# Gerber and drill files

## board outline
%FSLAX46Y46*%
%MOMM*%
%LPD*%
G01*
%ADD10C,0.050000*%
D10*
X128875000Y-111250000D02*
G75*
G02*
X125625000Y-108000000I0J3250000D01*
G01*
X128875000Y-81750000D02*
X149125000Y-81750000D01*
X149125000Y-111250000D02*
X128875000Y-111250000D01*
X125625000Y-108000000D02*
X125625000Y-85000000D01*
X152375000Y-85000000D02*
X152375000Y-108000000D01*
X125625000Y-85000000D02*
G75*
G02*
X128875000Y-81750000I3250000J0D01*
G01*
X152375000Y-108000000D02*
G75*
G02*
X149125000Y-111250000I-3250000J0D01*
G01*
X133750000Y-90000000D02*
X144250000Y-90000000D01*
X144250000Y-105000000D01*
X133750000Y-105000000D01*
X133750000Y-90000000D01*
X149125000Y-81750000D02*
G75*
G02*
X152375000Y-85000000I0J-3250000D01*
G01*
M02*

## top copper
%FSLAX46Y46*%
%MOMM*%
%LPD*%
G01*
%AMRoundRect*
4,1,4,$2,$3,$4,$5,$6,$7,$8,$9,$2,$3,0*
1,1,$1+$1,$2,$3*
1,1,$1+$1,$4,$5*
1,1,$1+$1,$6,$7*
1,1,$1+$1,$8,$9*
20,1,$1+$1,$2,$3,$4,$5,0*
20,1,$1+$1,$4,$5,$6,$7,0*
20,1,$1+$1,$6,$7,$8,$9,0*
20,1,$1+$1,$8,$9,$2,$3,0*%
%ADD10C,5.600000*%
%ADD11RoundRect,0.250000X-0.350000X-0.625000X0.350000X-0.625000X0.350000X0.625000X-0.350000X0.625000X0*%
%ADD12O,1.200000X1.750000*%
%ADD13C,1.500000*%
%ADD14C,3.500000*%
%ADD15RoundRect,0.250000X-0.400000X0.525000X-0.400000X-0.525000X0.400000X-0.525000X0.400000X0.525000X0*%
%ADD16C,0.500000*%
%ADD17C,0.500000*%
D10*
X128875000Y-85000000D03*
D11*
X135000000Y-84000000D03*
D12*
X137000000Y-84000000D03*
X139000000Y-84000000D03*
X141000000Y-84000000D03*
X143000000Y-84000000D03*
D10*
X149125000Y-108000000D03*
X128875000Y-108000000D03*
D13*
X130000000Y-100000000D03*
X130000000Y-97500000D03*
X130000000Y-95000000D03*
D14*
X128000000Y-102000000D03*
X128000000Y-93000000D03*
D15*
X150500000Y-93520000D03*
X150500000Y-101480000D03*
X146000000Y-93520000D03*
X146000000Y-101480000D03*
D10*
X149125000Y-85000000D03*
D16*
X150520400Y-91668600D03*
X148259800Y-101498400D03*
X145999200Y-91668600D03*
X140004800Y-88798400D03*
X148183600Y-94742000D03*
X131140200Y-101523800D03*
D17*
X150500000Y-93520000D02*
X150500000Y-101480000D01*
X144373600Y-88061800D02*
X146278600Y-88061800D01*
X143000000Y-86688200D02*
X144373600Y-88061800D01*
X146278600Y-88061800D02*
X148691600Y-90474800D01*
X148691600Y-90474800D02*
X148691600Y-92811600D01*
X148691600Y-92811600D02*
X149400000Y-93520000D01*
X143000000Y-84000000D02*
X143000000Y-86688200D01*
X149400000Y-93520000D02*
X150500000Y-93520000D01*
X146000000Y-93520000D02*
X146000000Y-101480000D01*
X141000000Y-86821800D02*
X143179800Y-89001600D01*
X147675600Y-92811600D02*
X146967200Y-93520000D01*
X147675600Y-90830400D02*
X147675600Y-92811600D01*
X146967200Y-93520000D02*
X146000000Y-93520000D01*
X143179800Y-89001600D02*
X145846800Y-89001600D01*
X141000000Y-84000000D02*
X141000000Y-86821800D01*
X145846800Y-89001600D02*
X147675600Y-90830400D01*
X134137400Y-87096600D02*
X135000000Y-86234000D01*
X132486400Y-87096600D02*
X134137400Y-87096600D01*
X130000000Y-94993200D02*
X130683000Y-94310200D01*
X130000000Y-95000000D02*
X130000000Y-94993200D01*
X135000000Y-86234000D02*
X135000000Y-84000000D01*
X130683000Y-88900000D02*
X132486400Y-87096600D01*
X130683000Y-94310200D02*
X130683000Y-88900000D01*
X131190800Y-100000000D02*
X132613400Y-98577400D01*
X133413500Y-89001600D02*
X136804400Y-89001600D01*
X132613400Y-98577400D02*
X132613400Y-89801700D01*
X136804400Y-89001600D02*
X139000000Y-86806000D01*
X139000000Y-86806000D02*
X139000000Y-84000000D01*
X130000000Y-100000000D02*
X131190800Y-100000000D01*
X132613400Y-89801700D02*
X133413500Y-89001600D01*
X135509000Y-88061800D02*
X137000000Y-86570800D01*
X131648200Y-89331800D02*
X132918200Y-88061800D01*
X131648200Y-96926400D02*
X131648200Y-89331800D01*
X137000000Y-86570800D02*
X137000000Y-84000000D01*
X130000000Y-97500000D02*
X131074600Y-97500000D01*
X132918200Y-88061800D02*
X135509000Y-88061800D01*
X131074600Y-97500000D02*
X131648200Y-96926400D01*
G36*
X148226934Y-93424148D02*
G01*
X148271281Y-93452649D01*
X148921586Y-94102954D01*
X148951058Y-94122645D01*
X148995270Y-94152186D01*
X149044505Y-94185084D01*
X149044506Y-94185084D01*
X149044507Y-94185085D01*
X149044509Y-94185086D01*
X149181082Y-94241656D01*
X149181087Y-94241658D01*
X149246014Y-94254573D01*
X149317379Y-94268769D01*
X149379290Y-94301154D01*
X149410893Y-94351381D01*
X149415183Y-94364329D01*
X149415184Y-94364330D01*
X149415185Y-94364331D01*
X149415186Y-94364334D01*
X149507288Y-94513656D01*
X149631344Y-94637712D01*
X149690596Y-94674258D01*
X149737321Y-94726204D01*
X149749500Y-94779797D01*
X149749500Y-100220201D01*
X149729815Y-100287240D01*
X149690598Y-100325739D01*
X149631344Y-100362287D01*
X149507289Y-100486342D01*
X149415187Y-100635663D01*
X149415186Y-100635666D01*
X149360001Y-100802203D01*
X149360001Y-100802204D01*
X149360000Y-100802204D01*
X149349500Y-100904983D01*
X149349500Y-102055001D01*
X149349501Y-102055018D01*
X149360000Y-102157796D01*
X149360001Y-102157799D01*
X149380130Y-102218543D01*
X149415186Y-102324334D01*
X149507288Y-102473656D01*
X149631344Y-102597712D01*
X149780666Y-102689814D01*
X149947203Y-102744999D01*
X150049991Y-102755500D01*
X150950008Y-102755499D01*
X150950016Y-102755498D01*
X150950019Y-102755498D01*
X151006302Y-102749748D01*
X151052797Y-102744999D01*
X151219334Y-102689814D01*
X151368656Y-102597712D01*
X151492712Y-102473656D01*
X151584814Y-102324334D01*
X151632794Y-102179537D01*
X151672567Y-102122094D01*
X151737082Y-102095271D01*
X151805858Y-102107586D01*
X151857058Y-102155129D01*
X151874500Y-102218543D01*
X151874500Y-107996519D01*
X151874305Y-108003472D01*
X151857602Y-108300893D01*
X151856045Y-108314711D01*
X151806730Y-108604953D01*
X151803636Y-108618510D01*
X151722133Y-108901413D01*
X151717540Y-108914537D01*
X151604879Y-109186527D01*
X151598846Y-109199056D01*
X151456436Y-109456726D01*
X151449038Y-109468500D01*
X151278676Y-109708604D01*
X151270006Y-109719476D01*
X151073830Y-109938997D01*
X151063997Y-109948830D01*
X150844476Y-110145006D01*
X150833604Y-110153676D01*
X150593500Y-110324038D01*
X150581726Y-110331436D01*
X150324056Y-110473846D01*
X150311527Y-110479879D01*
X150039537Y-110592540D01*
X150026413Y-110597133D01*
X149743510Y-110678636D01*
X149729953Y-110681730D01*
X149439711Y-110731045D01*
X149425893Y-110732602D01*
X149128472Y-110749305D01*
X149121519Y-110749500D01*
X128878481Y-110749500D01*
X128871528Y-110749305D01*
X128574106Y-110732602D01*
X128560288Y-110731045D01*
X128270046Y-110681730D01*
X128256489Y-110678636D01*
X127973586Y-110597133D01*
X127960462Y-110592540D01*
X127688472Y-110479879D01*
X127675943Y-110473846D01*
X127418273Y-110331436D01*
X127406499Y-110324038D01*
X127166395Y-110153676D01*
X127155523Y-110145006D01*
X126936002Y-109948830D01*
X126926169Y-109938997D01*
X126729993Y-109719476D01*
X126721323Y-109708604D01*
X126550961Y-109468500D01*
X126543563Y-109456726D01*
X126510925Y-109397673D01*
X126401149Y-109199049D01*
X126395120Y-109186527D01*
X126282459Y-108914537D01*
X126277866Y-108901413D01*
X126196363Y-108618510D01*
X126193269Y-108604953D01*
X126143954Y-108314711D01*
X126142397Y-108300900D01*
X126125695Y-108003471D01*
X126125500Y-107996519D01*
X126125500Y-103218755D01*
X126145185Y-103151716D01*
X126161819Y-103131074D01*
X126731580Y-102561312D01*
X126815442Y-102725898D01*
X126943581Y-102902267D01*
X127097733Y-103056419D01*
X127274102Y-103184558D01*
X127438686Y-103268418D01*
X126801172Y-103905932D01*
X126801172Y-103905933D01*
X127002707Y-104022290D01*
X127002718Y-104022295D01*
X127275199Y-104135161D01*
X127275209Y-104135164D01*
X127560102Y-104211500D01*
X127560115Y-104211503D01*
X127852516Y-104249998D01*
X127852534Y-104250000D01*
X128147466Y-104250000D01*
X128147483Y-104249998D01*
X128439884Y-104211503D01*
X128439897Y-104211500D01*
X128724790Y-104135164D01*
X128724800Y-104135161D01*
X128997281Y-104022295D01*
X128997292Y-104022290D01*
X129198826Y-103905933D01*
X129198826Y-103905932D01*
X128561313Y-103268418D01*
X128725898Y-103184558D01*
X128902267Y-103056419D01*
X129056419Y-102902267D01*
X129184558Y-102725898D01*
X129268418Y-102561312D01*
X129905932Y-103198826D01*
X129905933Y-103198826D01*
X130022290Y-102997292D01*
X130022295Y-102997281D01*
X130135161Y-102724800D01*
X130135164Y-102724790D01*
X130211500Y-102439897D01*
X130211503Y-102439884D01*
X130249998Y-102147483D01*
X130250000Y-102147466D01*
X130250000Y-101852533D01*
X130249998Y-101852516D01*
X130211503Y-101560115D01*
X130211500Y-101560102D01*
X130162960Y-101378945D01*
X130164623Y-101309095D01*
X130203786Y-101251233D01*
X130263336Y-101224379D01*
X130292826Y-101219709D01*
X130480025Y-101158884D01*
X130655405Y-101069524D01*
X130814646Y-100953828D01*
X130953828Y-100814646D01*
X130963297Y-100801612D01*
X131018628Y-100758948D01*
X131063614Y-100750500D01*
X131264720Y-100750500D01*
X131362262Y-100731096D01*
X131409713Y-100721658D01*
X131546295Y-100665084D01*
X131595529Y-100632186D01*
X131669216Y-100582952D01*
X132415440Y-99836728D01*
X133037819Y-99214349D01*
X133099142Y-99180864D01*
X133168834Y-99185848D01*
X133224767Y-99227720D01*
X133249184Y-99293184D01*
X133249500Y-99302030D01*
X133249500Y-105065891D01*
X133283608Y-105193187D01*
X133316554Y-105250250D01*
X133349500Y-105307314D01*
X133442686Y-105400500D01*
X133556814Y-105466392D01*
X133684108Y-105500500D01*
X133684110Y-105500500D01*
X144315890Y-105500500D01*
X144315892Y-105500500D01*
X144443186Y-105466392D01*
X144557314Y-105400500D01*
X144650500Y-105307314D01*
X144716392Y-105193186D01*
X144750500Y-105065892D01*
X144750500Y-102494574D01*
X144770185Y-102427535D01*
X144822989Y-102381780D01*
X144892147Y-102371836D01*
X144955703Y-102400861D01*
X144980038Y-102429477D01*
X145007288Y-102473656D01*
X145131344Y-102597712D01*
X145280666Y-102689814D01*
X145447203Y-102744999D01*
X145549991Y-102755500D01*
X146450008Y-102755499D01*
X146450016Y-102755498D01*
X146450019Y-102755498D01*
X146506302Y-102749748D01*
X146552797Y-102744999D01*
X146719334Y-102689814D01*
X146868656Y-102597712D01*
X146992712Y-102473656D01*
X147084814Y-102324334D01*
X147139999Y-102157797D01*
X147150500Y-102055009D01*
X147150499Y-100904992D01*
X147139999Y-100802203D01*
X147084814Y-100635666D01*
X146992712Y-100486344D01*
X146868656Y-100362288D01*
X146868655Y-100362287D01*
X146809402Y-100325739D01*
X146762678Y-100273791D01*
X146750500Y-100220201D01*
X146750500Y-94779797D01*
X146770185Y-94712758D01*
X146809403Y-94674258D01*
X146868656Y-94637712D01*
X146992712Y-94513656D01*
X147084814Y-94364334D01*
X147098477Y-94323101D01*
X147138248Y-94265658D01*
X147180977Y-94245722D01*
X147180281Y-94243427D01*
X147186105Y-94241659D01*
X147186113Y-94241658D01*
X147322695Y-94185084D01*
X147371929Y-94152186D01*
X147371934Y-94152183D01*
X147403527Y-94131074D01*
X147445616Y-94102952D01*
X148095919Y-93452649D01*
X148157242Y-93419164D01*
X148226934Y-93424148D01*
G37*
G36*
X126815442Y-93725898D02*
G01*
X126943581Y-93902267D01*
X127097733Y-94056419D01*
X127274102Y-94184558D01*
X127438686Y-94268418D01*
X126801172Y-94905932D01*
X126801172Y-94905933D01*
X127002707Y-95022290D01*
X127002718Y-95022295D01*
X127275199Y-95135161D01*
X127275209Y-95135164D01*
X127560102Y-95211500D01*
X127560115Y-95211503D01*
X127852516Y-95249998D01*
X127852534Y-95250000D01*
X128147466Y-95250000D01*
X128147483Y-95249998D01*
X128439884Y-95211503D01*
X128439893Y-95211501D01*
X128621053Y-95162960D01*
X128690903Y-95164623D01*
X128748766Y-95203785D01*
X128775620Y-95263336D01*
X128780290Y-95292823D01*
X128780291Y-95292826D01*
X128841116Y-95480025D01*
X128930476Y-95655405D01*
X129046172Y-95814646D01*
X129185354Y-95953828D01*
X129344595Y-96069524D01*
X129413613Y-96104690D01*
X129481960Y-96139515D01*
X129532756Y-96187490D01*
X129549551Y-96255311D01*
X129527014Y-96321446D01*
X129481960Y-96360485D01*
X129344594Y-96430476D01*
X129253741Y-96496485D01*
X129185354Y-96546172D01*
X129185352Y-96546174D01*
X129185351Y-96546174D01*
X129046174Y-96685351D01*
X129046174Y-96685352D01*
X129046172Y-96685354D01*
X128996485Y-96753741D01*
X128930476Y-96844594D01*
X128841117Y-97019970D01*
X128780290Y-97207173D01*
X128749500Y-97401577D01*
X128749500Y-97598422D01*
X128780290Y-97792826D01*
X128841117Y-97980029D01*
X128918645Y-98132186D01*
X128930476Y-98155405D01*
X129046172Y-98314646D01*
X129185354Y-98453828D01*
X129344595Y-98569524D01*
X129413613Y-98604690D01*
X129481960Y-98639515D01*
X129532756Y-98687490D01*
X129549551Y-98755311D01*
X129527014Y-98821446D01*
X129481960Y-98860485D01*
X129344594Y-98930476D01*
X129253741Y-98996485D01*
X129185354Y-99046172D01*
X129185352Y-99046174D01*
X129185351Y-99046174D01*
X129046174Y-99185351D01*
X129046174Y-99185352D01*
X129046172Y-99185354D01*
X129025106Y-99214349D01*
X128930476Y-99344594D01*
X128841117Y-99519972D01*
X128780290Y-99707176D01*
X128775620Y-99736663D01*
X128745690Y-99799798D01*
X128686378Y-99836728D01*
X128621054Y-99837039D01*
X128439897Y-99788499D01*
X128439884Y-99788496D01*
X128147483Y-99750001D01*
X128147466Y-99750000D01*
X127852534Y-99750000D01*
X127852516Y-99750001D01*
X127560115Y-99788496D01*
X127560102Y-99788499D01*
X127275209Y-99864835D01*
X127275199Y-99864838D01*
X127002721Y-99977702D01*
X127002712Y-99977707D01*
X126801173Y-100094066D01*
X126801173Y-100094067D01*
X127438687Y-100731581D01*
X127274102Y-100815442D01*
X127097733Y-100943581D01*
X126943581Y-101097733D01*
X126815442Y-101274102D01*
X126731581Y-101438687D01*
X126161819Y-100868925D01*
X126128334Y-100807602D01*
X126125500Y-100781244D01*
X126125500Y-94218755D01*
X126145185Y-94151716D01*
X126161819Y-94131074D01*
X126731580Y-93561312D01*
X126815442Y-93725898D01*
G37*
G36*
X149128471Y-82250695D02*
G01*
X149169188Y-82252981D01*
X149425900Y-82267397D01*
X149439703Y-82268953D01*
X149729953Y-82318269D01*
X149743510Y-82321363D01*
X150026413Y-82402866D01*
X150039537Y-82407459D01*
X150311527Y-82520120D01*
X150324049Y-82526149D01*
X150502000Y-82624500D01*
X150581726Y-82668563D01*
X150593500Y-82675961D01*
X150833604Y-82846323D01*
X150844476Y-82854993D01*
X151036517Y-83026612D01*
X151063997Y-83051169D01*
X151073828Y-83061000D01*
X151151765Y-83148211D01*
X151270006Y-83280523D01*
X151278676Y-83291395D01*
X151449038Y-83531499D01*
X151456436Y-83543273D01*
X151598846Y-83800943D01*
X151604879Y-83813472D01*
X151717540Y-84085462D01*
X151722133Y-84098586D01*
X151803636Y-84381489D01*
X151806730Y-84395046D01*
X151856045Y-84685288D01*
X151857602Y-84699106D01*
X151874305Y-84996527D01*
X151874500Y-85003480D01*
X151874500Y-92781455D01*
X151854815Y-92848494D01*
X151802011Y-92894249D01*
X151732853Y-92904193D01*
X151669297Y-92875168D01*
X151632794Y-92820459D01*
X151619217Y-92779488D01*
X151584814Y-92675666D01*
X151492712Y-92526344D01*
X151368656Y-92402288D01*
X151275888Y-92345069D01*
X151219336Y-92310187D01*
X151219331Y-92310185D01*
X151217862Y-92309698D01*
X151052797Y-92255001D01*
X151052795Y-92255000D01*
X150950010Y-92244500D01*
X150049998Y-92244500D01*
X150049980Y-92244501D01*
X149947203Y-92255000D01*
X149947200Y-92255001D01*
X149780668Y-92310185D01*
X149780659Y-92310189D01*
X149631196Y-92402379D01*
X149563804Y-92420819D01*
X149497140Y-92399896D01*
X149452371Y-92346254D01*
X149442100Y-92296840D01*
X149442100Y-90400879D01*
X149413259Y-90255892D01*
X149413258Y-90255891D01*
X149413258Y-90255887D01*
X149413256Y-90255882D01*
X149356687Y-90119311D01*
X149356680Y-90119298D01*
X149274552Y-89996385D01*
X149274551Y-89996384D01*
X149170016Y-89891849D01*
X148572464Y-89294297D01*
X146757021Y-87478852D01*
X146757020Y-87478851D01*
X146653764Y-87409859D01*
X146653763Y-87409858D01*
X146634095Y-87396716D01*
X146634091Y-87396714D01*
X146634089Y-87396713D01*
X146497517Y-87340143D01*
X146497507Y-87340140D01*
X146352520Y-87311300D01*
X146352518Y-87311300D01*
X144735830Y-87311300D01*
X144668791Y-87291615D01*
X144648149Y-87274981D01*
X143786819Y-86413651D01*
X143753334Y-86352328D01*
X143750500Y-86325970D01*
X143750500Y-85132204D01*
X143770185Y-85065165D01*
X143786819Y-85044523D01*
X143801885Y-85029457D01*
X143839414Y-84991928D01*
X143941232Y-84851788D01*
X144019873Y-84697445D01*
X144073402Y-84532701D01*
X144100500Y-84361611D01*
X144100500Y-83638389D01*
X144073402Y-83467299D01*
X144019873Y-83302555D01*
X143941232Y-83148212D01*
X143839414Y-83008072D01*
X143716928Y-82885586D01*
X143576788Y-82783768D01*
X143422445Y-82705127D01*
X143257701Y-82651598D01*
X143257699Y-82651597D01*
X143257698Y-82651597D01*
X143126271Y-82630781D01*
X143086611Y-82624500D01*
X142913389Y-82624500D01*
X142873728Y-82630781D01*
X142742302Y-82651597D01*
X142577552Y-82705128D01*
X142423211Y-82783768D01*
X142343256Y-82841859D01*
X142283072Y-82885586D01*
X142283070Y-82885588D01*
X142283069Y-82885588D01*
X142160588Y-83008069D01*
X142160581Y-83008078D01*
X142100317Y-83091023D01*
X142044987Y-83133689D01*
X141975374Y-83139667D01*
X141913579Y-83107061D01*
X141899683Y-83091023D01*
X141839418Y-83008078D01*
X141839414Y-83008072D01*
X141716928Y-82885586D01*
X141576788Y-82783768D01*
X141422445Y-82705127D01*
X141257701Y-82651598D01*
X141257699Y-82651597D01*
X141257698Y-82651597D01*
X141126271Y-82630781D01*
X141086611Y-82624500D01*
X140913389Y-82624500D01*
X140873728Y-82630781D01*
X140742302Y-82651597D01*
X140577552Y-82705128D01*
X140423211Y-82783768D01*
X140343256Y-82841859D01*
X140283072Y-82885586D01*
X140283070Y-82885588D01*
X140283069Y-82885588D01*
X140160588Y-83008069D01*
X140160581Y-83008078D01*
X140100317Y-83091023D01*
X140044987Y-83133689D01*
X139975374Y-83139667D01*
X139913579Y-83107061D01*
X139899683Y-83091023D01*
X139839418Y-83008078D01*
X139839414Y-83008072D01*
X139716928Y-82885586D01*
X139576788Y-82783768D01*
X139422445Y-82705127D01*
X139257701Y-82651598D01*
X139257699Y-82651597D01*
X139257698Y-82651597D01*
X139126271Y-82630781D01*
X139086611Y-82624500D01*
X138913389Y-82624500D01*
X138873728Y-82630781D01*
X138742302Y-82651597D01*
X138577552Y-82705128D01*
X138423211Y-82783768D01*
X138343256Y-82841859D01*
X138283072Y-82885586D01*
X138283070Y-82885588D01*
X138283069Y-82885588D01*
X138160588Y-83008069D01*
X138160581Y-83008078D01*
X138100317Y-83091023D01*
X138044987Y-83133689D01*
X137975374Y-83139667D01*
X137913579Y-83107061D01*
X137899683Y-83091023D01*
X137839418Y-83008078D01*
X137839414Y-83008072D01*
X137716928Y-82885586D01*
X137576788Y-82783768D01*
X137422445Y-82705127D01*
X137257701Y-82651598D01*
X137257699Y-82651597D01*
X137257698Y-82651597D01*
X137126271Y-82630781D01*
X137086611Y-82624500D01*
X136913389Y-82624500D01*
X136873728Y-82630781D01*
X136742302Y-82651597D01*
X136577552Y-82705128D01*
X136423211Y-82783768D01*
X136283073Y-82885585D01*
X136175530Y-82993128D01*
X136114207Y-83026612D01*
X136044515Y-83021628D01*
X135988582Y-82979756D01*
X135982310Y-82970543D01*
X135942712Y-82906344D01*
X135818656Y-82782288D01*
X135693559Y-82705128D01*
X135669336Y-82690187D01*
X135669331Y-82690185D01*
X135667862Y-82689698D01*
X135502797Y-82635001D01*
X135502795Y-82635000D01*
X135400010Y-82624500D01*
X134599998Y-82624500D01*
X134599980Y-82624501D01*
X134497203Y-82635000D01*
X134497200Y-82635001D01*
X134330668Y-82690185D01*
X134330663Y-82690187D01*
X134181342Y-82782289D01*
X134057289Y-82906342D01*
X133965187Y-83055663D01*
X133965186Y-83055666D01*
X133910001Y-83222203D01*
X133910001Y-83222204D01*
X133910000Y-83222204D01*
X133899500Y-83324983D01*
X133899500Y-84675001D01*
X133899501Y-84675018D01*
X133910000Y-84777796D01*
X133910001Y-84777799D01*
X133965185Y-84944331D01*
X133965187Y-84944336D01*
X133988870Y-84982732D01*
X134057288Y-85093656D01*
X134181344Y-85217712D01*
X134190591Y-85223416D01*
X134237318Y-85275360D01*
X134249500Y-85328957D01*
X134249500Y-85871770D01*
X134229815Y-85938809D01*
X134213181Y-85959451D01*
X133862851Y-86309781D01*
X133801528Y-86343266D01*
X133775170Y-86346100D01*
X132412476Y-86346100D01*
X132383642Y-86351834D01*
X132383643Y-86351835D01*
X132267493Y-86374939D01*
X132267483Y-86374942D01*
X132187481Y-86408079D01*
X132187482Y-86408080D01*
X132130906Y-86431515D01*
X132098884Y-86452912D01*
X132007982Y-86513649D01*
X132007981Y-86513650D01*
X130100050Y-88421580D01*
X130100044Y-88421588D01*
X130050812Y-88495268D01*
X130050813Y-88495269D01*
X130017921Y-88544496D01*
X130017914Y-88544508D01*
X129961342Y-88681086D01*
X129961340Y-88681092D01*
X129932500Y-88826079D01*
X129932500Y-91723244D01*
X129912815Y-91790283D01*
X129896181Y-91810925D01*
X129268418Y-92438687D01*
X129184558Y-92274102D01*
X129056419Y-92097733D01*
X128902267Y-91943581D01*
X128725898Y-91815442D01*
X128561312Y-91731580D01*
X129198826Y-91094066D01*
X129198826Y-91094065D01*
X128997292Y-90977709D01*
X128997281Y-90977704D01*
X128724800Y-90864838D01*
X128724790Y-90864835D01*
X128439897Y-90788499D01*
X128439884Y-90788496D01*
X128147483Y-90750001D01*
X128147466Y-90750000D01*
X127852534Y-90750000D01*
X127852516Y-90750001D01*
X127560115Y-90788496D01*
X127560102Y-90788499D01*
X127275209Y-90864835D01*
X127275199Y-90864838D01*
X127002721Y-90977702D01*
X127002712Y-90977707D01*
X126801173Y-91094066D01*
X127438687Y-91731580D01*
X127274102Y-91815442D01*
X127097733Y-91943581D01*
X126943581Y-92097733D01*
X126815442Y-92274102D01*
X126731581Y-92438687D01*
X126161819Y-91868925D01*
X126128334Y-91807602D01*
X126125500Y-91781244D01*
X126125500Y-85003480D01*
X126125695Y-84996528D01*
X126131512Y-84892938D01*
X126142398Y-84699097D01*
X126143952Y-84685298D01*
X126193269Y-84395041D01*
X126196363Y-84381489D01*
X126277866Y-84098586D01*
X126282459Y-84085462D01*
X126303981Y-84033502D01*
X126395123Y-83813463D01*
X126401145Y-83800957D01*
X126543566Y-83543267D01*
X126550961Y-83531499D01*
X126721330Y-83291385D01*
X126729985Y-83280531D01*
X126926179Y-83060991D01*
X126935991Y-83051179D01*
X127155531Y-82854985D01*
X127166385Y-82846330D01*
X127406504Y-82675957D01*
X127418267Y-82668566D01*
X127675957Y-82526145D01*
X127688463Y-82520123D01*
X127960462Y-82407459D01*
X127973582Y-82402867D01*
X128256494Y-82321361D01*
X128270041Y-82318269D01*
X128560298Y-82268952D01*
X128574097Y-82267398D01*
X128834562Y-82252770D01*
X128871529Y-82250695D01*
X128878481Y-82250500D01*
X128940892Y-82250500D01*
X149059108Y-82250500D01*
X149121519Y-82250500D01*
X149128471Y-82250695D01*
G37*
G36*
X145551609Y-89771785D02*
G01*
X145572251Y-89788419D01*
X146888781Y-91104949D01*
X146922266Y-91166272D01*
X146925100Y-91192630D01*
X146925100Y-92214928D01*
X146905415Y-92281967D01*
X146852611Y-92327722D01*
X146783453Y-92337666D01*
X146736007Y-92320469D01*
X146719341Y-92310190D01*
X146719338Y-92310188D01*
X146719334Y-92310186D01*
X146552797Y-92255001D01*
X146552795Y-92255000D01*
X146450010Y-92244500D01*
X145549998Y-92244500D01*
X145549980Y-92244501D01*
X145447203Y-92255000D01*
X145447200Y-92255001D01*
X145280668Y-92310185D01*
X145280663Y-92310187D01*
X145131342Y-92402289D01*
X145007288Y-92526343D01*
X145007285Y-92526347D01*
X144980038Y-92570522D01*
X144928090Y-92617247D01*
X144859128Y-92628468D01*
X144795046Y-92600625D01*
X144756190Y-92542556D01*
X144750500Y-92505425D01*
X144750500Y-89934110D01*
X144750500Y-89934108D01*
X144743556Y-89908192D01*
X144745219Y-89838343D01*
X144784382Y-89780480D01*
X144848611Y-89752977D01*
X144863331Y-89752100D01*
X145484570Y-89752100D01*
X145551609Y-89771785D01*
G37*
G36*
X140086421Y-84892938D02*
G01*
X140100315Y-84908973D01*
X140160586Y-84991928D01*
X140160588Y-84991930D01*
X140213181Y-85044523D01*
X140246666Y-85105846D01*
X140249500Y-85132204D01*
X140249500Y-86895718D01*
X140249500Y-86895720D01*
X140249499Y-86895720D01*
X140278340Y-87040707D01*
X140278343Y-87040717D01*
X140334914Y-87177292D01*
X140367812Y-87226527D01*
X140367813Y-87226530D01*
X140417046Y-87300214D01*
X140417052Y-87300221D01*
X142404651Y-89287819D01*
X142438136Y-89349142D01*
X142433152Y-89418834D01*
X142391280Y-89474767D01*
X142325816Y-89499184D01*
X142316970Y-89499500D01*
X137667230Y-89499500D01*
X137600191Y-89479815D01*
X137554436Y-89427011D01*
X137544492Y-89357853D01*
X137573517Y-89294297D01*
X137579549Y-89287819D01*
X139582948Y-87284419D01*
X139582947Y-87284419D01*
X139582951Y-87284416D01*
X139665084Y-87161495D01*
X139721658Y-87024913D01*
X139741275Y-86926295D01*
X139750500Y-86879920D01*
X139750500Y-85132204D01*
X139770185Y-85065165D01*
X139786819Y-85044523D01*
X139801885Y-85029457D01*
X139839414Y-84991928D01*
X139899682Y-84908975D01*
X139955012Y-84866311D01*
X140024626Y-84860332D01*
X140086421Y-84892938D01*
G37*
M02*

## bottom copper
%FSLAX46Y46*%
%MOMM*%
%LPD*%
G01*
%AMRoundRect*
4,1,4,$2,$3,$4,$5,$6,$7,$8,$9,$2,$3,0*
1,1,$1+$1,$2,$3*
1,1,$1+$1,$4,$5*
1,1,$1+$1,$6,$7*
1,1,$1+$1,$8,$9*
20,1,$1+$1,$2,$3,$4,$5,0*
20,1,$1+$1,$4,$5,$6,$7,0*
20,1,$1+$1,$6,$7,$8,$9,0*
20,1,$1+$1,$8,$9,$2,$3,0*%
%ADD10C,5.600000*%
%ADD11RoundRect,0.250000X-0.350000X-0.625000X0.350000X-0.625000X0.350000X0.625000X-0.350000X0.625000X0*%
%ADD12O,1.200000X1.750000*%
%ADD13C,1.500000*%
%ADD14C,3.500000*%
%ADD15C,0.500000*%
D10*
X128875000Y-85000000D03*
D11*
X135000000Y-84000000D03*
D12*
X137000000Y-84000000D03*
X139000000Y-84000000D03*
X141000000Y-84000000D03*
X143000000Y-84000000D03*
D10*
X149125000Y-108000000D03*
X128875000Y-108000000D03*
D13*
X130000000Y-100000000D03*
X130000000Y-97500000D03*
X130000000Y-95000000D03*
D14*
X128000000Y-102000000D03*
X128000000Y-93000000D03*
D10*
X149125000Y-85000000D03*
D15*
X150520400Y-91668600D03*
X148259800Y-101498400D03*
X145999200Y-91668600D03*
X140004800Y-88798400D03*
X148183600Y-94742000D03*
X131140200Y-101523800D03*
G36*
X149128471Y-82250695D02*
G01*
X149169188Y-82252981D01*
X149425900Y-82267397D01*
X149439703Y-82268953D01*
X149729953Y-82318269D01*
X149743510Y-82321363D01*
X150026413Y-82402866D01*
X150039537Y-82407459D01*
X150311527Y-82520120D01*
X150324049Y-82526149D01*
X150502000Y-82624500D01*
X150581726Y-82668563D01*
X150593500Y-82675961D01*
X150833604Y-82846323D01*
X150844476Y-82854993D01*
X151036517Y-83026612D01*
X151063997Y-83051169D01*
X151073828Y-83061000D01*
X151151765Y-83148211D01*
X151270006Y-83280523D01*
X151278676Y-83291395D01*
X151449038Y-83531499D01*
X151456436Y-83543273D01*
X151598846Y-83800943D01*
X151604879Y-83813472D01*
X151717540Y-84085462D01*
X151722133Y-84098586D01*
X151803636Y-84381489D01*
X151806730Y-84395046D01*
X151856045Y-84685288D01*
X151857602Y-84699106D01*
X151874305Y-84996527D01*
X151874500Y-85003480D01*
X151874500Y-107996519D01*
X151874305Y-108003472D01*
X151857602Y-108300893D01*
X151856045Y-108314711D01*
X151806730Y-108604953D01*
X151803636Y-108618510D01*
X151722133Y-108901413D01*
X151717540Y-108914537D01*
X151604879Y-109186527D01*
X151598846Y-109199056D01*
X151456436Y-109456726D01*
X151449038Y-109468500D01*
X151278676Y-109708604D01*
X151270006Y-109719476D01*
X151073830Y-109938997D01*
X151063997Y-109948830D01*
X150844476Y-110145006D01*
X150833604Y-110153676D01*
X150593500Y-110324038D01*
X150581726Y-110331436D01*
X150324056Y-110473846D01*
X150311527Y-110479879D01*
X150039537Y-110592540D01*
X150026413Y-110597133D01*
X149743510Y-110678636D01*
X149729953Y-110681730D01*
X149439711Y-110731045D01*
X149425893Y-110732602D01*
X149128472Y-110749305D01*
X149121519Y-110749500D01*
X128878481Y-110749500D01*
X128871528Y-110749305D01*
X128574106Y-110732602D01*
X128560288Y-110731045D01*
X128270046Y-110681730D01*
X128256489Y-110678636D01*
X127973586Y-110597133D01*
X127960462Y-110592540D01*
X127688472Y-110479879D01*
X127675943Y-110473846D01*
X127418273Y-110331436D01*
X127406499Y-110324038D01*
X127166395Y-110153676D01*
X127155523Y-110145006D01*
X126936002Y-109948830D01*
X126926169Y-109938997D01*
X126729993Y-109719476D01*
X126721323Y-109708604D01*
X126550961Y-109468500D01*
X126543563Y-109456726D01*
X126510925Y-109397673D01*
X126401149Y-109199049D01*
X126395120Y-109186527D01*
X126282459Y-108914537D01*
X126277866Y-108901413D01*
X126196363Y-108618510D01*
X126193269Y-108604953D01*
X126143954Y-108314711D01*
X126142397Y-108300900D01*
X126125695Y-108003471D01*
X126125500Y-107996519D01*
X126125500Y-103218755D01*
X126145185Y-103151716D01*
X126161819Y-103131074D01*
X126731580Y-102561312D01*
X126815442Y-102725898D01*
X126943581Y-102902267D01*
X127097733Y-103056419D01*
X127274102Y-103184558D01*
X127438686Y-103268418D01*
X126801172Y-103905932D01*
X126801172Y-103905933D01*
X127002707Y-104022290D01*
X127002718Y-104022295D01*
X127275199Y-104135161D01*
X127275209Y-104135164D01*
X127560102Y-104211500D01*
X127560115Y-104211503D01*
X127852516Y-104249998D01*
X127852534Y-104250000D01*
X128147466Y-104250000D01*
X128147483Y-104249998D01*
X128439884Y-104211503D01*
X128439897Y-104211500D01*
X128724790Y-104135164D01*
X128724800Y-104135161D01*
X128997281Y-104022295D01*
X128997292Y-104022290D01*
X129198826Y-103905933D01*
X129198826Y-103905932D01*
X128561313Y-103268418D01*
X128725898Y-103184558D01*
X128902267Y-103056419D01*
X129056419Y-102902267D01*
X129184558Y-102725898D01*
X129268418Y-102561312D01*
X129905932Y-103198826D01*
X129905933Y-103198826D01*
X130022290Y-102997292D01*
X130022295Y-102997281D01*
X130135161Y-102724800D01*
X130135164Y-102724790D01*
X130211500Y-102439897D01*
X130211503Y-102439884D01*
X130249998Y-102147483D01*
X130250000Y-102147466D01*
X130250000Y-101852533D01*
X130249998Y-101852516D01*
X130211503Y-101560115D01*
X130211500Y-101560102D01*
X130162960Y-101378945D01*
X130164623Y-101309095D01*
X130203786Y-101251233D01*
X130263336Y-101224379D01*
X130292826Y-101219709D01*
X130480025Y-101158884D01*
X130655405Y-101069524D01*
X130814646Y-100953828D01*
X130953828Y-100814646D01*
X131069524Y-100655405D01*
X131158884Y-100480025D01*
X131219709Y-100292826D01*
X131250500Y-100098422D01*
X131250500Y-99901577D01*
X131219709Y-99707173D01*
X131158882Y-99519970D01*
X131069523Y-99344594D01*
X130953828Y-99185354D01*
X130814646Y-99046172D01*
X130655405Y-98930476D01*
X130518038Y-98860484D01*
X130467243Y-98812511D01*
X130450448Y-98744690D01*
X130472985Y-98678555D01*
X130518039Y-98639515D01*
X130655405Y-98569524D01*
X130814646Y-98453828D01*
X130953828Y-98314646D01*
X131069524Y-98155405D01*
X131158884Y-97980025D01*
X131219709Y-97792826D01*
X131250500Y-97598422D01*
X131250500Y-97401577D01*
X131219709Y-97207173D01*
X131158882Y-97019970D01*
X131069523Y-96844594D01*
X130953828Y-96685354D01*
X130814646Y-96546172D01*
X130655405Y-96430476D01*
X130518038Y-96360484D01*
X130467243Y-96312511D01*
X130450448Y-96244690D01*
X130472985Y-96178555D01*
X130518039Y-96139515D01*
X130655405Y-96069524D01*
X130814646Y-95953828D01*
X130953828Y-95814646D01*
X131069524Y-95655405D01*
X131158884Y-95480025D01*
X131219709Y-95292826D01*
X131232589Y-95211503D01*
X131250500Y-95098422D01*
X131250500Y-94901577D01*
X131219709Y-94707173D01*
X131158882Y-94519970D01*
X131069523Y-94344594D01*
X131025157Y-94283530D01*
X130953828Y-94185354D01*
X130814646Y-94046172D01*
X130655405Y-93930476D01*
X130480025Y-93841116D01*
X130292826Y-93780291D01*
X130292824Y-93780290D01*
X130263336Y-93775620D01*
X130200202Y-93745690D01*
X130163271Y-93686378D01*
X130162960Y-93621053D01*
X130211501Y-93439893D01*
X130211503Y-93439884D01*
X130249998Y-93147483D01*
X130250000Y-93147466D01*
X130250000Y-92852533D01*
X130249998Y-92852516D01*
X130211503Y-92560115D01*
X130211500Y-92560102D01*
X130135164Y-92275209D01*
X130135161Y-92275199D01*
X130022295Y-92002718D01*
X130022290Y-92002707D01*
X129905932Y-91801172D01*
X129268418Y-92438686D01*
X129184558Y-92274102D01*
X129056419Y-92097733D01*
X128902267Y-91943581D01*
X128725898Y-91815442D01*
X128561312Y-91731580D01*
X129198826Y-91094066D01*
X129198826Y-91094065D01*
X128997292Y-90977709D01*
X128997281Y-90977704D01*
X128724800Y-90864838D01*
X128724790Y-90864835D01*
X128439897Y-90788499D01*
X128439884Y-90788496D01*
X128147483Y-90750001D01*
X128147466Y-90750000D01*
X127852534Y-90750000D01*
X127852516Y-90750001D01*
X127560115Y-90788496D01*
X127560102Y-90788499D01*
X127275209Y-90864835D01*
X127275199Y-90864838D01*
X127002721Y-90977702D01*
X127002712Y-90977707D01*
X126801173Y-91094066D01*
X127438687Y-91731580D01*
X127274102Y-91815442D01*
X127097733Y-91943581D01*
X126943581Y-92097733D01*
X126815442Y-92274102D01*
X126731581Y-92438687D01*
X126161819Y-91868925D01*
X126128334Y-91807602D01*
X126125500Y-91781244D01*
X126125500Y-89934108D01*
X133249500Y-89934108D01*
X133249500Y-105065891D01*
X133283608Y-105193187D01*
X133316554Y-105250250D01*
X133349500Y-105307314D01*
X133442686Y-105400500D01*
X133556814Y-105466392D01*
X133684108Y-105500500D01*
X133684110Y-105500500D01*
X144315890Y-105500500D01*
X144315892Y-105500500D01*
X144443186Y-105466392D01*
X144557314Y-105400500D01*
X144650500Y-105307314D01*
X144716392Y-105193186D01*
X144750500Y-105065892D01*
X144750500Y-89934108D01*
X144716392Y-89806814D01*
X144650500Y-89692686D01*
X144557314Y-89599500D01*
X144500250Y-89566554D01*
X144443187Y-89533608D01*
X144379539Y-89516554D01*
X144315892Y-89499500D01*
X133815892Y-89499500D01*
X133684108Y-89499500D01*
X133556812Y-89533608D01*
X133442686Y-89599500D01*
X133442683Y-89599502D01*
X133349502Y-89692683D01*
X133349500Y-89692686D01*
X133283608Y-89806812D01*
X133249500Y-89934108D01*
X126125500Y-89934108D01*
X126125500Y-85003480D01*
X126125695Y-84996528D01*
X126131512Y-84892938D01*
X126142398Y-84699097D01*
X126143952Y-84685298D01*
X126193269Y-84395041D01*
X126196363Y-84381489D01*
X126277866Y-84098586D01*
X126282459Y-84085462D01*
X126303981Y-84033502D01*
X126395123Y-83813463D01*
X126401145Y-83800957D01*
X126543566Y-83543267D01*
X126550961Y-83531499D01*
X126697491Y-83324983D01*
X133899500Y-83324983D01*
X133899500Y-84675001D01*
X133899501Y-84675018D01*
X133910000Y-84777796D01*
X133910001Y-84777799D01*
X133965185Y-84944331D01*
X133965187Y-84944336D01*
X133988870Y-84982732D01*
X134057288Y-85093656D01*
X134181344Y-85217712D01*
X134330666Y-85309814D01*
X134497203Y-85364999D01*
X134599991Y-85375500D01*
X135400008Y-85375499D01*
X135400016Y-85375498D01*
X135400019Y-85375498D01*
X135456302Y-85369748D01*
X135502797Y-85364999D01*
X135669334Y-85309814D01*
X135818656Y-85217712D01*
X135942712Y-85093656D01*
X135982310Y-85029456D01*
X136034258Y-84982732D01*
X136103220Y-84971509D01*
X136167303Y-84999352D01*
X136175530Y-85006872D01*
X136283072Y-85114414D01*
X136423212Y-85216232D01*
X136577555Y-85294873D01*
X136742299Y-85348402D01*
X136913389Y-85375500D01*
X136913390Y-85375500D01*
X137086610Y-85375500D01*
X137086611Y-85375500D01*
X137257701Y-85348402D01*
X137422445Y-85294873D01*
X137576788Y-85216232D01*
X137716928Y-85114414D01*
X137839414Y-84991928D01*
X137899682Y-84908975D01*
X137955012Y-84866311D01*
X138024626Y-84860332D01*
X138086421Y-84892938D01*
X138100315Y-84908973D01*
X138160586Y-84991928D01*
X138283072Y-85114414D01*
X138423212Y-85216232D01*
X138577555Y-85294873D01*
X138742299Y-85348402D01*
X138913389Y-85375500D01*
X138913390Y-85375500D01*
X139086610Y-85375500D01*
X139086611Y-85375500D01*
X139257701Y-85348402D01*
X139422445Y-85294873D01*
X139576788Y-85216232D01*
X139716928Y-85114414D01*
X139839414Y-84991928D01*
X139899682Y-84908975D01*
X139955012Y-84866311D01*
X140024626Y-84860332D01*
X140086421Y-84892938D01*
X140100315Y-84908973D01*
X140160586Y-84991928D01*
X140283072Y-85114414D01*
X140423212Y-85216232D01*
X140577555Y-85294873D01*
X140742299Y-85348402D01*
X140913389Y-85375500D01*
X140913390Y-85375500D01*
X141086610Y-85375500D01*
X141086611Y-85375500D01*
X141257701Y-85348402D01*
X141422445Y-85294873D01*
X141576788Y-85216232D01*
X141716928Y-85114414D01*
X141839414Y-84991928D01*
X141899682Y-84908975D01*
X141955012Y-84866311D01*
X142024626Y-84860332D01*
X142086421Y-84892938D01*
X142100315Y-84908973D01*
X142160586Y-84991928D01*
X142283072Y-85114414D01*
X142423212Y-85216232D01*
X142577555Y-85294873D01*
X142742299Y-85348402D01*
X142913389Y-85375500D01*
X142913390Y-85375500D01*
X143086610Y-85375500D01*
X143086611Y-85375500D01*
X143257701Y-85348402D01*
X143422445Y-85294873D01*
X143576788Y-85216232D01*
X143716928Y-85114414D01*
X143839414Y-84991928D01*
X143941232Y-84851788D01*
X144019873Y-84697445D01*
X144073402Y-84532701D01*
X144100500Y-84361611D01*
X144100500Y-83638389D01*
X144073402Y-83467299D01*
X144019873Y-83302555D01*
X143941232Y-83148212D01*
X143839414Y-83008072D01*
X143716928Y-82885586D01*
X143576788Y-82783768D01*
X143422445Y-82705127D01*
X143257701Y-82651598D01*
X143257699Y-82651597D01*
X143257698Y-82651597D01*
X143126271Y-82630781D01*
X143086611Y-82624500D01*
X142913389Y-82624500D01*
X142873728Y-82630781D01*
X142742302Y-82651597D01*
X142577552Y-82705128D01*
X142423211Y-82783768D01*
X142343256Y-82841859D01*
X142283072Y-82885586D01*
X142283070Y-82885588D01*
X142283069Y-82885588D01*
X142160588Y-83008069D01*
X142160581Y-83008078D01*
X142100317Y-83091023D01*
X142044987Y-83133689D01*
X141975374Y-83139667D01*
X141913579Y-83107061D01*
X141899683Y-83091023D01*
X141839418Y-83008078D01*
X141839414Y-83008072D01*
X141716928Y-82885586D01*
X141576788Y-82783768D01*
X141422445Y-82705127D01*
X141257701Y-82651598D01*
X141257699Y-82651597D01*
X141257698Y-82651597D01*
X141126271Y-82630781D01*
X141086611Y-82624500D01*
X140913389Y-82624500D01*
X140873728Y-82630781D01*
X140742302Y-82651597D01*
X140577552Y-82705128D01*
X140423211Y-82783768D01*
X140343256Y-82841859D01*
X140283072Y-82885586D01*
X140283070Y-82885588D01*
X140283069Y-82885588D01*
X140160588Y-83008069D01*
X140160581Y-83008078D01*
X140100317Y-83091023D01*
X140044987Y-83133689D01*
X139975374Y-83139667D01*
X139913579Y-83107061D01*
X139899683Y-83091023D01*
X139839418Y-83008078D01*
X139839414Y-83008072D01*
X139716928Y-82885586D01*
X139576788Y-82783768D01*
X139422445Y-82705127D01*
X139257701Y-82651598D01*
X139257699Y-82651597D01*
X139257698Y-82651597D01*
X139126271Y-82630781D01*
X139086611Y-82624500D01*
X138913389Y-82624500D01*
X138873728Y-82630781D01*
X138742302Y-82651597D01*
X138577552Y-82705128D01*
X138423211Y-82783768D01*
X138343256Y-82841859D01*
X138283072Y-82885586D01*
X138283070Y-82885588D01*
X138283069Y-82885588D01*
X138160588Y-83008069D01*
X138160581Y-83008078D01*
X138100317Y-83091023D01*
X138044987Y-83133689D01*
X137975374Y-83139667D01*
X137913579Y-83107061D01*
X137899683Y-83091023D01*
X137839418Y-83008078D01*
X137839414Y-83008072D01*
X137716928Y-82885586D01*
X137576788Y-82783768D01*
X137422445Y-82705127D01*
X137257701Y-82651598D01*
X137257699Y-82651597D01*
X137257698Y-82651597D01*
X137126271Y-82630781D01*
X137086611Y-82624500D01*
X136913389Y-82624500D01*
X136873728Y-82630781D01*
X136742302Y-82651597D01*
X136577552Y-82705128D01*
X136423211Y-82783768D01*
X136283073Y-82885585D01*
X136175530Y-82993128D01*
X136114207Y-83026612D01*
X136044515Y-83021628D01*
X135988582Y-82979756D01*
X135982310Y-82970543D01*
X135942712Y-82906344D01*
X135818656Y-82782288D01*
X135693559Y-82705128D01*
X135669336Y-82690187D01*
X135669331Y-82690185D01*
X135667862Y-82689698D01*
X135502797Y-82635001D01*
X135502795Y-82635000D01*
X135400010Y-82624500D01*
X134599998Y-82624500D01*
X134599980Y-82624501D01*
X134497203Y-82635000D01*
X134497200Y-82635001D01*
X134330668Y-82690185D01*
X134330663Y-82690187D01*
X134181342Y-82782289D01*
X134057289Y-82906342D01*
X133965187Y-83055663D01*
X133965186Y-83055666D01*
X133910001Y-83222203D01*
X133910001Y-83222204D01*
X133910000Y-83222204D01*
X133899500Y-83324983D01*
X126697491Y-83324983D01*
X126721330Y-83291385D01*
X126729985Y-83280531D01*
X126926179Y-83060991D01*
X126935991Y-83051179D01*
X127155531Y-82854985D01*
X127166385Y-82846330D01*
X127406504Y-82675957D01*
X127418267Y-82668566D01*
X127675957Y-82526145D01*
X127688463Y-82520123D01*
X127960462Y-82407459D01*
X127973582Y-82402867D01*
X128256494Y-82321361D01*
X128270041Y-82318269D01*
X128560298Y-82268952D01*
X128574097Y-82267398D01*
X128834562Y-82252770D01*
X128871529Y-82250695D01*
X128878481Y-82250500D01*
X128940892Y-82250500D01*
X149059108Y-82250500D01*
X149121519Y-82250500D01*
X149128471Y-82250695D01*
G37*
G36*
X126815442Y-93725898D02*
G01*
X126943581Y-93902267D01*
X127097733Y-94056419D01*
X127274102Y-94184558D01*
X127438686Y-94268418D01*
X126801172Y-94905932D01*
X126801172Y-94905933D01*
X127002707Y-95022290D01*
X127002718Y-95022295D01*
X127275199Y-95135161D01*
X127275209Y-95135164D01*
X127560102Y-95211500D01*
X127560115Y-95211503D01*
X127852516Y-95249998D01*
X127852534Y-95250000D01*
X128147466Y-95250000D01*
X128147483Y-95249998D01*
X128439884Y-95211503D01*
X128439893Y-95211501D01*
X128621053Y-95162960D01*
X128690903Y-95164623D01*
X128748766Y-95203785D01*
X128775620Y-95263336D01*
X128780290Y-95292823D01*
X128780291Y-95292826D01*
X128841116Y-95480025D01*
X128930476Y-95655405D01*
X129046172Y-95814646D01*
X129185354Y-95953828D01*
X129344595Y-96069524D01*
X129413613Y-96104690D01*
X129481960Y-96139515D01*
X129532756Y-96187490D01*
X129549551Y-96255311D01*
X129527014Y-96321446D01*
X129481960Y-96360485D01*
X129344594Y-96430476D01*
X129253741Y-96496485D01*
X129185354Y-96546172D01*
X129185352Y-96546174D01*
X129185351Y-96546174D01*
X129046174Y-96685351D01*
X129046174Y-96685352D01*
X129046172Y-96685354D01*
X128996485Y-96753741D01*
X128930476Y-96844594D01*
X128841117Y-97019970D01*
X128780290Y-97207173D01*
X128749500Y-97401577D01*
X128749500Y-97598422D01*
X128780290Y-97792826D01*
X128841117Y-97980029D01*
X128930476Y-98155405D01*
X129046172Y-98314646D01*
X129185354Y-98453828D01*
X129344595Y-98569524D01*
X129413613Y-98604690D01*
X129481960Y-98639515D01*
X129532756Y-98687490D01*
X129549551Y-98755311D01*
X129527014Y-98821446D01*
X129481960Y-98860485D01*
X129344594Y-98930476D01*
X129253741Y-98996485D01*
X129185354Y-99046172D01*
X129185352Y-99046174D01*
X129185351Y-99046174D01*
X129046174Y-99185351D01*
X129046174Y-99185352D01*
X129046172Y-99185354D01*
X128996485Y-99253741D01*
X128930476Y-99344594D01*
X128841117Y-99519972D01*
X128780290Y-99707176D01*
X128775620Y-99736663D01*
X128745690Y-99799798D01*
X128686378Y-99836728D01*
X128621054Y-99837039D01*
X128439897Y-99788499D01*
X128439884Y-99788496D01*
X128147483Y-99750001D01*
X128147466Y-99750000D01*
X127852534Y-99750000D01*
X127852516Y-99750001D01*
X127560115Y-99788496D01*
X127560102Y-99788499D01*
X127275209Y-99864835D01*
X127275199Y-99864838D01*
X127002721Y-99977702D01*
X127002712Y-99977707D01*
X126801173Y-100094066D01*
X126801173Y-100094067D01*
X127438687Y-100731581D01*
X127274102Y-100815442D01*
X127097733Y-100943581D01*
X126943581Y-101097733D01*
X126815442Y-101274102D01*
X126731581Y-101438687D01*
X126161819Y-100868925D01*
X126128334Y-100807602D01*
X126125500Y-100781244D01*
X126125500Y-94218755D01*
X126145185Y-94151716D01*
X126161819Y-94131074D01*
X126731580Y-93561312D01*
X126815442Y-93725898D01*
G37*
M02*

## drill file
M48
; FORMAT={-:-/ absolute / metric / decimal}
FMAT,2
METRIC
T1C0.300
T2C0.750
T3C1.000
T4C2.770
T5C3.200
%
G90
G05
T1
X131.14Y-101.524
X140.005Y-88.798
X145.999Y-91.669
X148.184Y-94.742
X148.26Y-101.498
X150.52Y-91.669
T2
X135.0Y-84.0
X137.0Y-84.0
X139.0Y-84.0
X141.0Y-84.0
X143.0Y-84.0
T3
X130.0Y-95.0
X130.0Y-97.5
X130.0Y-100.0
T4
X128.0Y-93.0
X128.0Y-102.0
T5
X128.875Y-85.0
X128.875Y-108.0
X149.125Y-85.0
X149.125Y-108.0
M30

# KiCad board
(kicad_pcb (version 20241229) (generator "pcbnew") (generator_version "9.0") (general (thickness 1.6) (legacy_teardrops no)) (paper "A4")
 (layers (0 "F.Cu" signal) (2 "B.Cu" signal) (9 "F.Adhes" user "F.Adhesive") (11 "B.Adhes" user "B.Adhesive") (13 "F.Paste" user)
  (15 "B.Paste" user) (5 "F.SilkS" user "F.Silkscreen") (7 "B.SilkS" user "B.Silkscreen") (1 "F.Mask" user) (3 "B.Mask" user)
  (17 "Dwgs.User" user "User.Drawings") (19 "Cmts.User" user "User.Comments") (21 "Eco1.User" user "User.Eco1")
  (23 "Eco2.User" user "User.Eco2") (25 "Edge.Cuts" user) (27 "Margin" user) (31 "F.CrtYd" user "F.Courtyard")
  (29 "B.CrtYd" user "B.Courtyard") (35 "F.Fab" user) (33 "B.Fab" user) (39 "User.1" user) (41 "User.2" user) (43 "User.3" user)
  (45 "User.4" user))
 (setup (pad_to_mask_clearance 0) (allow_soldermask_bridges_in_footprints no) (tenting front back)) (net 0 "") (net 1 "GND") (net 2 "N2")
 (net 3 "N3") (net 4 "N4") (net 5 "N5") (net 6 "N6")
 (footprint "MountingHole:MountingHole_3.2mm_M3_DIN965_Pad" (layer "F.Cu") (at 128.875 85)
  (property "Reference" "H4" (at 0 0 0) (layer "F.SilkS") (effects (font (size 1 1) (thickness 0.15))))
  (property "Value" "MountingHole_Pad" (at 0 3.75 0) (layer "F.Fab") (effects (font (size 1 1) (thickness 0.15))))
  (pad "1" thru_hole circle (at 0 0) (size 5.6 5.6) (drill 3.2) (layers "*.Cu" "*.Mask") (remove_unused_layers no) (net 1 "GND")
   (zone_connect 2)))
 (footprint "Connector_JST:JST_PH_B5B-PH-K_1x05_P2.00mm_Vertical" (layer "F.Cu") (at 135 84)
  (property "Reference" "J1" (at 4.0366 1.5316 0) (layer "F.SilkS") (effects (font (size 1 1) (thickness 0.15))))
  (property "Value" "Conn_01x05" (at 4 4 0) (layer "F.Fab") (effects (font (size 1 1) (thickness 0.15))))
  (pad "1" thru_hole roundrect (at 0 0) (size 1.2 1.75) (drill 0.75) (layers "*.Cu" "*.Mask") (remove_unused_layers no)
   (roundrect_rratio 0.208333) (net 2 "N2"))
  (pad "2" thru_hole oval (at 2 0) (size 1.2 1.75) (drill 0.75) (layers "*.Cu" "*.Mask") (remove_unused_layers no) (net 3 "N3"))
  (pad "3" thru_hole oval (at 4 0) (size 1.2 1.75) (drill 0.75) (layers "*.Cu" "*.Mask") (remove_unused_layers no) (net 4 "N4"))
  (pad "4" thru_hole oval (at 6 0) (size 1.2 1.75) (drill 0.75) (layers "*.Cu" "*.Mask") (remove_unused_layers no) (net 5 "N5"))
  (pad "5" thru_hole oval (at 8 0) (size 1.2 1.75) (drill 0.75) (layers "*.Cu" "*.Mask") (remove_unused_layers no) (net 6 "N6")))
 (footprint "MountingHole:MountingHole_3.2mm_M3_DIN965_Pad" (layer "F.Cu") (at 149.125 108)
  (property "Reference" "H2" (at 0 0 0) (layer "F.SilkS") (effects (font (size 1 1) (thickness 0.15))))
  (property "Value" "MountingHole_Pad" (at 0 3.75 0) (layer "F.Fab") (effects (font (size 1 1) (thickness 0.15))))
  (pad "1" thru_hole circle (at 0 0) (size 5.6 5.6) (drill 3.2) (layers "*.Cu" "*.Mask") (remove_unused_layers no) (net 1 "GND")
   (zone_connect 2)))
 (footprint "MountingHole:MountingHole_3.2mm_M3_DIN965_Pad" (layer "F.Cu") (at 128.875 108)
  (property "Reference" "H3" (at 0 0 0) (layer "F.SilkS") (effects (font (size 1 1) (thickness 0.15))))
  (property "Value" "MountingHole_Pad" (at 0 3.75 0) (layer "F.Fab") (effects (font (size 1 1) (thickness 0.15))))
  (pad "1" thru_hole circle (at 0 0) (size 5.6 5.6) (drill 3.2) (layers "*.Cu" "*.Mask") (remove_unused_layers no) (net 1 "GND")
   (zone_connect 2)))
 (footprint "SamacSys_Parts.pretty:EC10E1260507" (layer "F.Cu") (at 130 100 90)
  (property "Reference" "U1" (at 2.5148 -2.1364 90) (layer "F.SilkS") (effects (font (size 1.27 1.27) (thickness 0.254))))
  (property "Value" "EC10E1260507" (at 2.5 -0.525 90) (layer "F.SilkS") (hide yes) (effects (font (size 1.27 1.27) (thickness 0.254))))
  (pad "A1" thru_hole circle (at 0 0 90) (size 1.5 1.5) (drill 1) (layers "*.Cu" "*.Mask") (remove_unused_layers no) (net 4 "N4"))
  (pad "B1" thru_hole circle (at 2.5 0 90) (size 1.5 1.5) (drill 1) (layers "*.Cu" "*.Mask") (remove_unused_layers no) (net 3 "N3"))
  (pad "C1" thru_hole circle (at 5 0 90) (size 1.5 1.5) (drill 1) (layers "*.Cu" "*.Mask") (remove_unused_layers no) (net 2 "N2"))
  (pad "MH1" thru_hole circle (at -2 -2 90) (size 3.5 3.5) (drill 2.77) (layers "*.Cu" "*.Mask") (remove_unused_layers no) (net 1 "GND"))
  (pad "MH2" thru_hole circle (at 7 -2 90) (size 3.5 3.5) (drill 2.77) (layers "*.Cu" "*.Mask") (remove_unused_layers no) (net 1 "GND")))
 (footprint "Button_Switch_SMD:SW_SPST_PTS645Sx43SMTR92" (layer "F.Cu") (at 148.25 97.5 -90)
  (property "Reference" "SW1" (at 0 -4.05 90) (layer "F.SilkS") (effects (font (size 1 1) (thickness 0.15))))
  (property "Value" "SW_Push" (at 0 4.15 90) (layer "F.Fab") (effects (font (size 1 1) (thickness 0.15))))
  (pad "1" smd roundrect (at -3.98 -2.25 270) (size 1.55 1.3) (layers "F.Cu" "F.Mask" "F.Paste") (roundrect_rratio 0.1923076923)
   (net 6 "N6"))
  (pad "1" smd roundrect (at 3.98 -2.25 270) (size 1.55 1.3) (layers "F.Cu" "F.Mask" "F.Paste") (roundrect_rratio 0.1923076923) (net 6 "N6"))
  (pad "2" smd roundrect (at -3.98 2.25 270) (size 1.55 1.3) (layers "F.Cu" "F.Mask" "F.Paste") (roundrect_rratio 0.1923076923) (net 5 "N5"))
  (pad "2" smd roundrect (at 3.98 2.25 270) (size 1.55 1.3) (layers "F.Cu" "F.Mask" "F.Paste") (roundrect_rratio 0.1923076923) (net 5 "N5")))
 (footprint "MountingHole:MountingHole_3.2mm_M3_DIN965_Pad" (layer "F.Cu") (at 149.125 85)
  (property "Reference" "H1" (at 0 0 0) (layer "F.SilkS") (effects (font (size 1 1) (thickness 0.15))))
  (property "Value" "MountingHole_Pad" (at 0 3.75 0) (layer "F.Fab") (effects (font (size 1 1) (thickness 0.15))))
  (pad "1" thru_hole circle (at 0 0) (size 5.6 5.6) (drill 3.2) (layers "*.Cu" "*.Mask") (remove_unused_layers no) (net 1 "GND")
   (zone_connect 2)))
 (gr_arc (start 128.875 111.25) (mid 126.576903 110.298097) (end 125.625 108) (stroke (width 0.05) (type solid)) (layer "Edge.Cuts"))
 (gr_line (start 128.875 81.75) (end 149.125 81.75) (stroke (width 0.05) (type solid)) (layer "Edge.Cuts"))
 (gr_line (start 149.125 111.25) (end 128.875 111.25) (stroke (width 0.05) (type default)) (layer "Edge.Cuts"))
 (gr_line (start 125.625 108) (end 125.625 85) (stroke (width 0.05) (type default)) (layer "Edge.Cuts"))
 (gr_line (start 152.375 85) (end 152.375 108) (stroke (width 0.05) (type solid)) (layer "Edge.Cuts"))
 (gr_arc (start 125.625 85) (mid 126.576903 82.701903) (end 128.875 81.75) (stroke (width 0.05) (type solid)) (layer "Edge.Cuts"))
 (gr_arc (start 152.375 108) (mid 151.423097 110.298097) (end 149.125 111.25) (stroke (width 0.05) (type solid)) (layer "Edge.Cuts"))
 (gr_rect (start 133.75 90) (end 144.25 105) (stroke (width 0.05) (type solid)) (fill no) (layer "Edge.Cuts"))
 (gr_arc (start 149.125 81.75) (mid 151.423097 82.701903) (end 152.375 85) (stroke (width 0.05) (type solid)) (layer "Edge.Cuts"))
 (segment (start 150.5 93.52) (end 150.5 101.48) (width 0.5) (layer "F.Cu") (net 6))
 (segment (start 144.3736 88.0618) (end 146.2786 88.0618) (width 0.5) (layer "F.Cu") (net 6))
 (segment (start 143 86.6882) (end 144.3736 88.0618) (width 0.5) (layer "F.Cu") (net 6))
 (segment (start 146.2786 88.0618) (end 148.6916 90.4748) (width 0.5) (layer "F.Cu") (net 6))
 (segment (start 148.6916 90.4748) (end 148.6916 92.8116) (width 0.5) (layer "F.Cu") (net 6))
 (segment (start 148.6916 92.8116) (end 149.4 93.52) (width 0.5) (layer "F.Cu") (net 6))
 (segment (start 143 84) (end 143 86.6882) (width 0.5) (layer "F.Cu") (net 6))
 (segment (start 149.4 93.52) (end 150.5 93.52) (width 0.5) (layer "F.Cu") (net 6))
 (segment (start 146 93.52) (end 146 101.48) (width 0.5) (layer "F.Cu") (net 5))
 (segment (start 141 86.8218) (end 143.1798 89.0016) (width 0.5) (layer "F.Cu") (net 5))
 (segment (start 147.6756 92.8116) (end 146.9672 93.52) (width 0.5) (layer "F.Cu") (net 5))
 (segment (start 147.6756 90.8304) (end 147.6756 92.8116) (width 0.5) (layer "F.Cu") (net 5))
 (segment (start 146.9672 93.52) (end 146 93.52) (width 0.5) (layer "F.Cu") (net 5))
 (segment (start 143.1798 89.0016) (end 145.8468 89.0016) (width 0.5) (layer "F.Cu") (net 5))
 (segment (start 141 84) (end 141 86.8218) (width 0.5) (layer "F.Cu") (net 5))
 (segment (start 145.8468 89.0016) (end 147.6756 90.8304) (width 0.5) (layer "F.Cu") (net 5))
 (segment (start 134.1374 87.0966) (end 135 86.234) (width 0.5) (layer "F.Cu") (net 2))
 (segment (start 132.4864 87.0966) (end 134.1374 87.0966) (width 0.5) (layer "F.Cu") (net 2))
 (segment (start 130 94.9932) (end 130.683 94.3102) (width 0.5) (layer "F.Cu") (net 2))
 (segment (start 130 95) (end 130 94.9932) (width 0.5) (layer "F.Cu") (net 2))
 (segment (start 135 86.234) (end 135 84) (width 0.5) (layer "F.Cu") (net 2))
 (segment (start 130.683 88.9) (end 132.4864 87.0966) (width 0.5) (layer "F.Cu") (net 2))
 (segment (start 130.683 94.3102) (end 130.683 88.9) (width 0.5) (layer "F.Cu") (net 2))
 (segment (start 131.1908 100) (end 132.6134 98.5774) (width 0.5) (layer "F.Cu") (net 4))
 (segment (start 133.4135 89.0016) (end 136.8044 89.0016) (width 0.5) (layer "F.Cu") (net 4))
 (segment (start 132.6134 98.5774) (end 132.6134 89.8017) (width 0.5) (layer "F.Cu") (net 4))
 (segment (start 136.8044 89.0016) (end 139 86.806) (width 0.5) (layer "F.Cu") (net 4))
 (segment (start 139 86.806) (end 139 84) (width 0.5) (layer "F.Cu") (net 4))
 (segment (start 130 100) (end 131.1908 100) (width 0.5) (layer "F.Cu") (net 4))
 (segment (start 132.6134 89.8017) (end 133.4135 89.0016) (width 0.5) (layer "F.Cu") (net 4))
 (segment (start 135.509 88.0618) (end 137 86.5708) (width 0.5) (layer "F.Cu") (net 3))
 (segment (start 131.6482 89.3318) (end 132.9182 88.0618) (width 0.5) (layer "F.Cu") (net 3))
 (segment (start 131.6482 96.9264) (end 131.6482 89.3318) (width 0.5) (layer "F.Cu") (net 3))
 (segment (start 137 86.5708) (end 137 84) (width 0.5) (layer "F.Cu") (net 3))
 (segment (start 130 97.5) (end 131.0746 97.5) (width 0.5) (layer "F.Cu") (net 3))
 (segment (start 132.9182 88.0618) (end 135.509 88.0618) (width 0.5) (layer "F.Cu") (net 3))
 (segment (start 131.0746 97.5) (end 131.6482 96.9264) (width 0.5) (layer "F.Cu") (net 3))
 (via (at 150.5204 91.6686) (size 0.5) (drill 0.3) (layers "F.Cu" "B.Cu") (free yes) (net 1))
 (via (at 148.2598 101.4984) (size 0.5) (drill 0.3) (layers "F.Cu" "B.Cu") (free yes) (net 1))
 (via (at 145.9992 91.6686) (size 0.5) (drill 0.3) (layers "F.Cu" "B.Cu") (free yes) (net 1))
 (via (at 140.0048 88.7984) (size 0.5) (drill 0.3) (layers "F.Cu" "B.Cu") (free yes) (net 1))
 (via (at 148.1836 94.742) (size 0.5) (drill 0.3) (layers "F.Cu" "B.Cu") (free yes) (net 1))
 (via (at 131.1402 101.5238) (size 0.5) (drill 0.3) (layers "F.Cu" "B.Cu") (free yes) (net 1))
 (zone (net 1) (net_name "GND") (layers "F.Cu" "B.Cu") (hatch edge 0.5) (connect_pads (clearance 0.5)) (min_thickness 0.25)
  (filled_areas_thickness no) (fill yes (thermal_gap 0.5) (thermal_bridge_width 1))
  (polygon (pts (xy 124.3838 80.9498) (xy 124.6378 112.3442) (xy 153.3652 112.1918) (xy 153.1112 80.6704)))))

